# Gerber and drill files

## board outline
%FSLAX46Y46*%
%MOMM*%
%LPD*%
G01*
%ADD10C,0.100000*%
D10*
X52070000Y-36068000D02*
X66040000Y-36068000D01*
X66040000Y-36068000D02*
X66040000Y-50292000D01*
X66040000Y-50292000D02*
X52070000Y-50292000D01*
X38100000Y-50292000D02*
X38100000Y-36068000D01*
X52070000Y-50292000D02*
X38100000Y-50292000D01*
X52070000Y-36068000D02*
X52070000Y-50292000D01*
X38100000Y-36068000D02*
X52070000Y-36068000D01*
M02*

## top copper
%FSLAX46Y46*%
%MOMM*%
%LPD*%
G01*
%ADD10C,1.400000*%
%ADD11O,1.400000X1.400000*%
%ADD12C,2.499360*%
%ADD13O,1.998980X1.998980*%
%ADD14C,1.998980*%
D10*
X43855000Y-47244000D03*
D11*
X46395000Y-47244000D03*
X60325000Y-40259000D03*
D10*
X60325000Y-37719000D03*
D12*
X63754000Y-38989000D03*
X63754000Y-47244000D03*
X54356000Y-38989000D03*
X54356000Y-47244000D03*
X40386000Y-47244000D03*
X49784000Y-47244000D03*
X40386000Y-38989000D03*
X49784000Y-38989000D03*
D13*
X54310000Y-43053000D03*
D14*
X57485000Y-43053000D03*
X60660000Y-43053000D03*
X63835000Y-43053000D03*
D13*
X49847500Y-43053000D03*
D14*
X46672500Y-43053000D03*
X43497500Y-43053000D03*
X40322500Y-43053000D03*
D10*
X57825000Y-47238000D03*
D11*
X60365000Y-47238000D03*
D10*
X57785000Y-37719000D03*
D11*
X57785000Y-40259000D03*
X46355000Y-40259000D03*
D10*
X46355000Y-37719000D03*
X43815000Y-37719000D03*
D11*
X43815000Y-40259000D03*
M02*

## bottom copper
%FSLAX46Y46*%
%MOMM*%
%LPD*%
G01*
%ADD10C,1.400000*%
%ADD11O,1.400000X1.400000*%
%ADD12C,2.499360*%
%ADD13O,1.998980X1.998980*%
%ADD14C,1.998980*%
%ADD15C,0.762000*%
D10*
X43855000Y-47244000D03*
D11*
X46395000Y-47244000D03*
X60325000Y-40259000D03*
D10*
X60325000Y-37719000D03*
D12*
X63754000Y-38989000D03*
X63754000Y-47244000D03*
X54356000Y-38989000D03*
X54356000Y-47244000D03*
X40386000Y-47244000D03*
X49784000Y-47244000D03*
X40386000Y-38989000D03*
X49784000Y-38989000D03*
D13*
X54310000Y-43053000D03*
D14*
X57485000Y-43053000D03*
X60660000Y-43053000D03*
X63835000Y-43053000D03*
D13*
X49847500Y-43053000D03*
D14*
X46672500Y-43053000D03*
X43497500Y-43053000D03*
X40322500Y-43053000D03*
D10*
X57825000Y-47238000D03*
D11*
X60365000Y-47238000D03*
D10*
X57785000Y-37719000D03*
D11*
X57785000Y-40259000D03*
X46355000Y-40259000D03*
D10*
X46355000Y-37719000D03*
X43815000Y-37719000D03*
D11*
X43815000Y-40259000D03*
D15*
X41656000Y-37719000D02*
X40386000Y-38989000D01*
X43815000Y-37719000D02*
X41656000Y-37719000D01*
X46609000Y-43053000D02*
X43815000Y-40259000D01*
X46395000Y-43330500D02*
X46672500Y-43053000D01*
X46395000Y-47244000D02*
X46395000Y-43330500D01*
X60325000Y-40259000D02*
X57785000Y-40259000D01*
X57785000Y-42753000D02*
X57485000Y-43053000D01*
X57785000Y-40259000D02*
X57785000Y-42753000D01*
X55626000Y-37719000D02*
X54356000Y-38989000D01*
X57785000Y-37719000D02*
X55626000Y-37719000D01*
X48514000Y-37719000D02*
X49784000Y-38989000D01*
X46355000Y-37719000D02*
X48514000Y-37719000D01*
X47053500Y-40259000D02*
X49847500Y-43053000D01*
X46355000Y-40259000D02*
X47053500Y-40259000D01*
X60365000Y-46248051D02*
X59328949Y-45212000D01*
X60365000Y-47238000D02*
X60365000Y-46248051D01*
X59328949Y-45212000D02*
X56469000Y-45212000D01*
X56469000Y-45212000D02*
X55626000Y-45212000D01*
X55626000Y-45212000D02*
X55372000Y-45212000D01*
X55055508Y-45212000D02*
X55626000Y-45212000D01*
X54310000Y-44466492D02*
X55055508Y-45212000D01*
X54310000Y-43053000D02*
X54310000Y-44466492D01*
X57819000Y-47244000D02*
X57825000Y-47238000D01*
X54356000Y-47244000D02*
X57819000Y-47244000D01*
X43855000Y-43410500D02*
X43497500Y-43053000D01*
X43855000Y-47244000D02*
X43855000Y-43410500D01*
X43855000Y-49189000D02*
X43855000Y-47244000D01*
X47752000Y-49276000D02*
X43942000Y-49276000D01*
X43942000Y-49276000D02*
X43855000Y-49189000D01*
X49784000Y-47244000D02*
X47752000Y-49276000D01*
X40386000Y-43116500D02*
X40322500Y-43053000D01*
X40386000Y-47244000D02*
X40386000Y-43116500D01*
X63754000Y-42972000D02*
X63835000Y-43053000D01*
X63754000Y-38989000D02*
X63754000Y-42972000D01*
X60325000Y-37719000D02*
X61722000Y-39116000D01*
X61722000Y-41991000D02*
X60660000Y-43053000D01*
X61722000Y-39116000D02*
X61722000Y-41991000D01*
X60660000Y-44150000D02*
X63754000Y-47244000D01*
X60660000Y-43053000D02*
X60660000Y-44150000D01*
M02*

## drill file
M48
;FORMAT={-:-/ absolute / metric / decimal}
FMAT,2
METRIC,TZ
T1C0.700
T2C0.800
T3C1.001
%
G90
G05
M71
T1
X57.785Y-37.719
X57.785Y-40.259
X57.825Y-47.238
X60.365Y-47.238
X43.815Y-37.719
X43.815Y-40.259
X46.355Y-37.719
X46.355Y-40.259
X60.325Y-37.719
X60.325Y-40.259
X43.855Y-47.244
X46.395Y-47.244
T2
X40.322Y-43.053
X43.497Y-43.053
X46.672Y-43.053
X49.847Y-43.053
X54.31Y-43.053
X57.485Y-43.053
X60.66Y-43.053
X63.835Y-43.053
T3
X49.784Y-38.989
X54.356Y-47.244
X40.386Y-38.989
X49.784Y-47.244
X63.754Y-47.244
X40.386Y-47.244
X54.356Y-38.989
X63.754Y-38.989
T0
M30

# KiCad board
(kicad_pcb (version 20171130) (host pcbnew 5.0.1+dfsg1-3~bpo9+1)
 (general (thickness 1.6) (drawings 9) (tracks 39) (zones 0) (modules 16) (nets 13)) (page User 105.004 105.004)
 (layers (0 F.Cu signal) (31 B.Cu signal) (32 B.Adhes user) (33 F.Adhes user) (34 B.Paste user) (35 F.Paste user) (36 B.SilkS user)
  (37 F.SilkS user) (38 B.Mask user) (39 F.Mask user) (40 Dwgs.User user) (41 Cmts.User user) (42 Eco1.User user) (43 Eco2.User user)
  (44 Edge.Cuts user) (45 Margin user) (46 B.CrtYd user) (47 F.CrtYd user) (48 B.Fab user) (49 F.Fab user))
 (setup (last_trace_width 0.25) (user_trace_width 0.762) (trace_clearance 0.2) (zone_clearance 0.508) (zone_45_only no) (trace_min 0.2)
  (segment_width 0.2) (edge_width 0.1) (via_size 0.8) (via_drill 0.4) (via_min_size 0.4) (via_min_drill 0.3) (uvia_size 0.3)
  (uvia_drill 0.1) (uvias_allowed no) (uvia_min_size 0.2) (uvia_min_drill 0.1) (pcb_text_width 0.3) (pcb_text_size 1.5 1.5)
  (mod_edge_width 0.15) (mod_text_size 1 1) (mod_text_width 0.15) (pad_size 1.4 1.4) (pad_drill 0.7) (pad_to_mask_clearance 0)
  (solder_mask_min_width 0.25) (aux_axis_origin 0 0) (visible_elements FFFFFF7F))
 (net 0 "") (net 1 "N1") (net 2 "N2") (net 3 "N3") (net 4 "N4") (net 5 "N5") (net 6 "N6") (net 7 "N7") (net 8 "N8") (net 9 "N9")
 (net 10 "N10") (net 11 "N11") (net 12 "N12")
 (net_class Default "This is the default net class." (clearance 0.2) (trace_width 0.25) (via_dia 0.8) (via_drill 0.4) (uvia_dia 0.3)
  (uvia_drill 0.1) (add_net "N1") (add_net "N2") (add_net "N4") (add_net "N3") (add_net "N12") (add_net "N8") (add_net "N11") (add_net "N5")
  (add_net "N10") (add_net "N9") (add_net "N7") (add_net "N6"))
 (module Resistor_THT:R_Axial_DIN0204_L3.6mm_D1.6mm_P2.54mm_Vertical (layer F.Cu) (at 43.855 47.244)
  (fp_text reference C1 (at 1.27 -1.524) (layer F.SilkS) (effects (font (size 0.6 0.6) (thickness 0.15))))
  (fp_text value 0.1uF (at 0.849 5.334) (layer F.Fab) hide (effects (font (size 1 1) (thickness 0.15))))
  (pad 1 thru_hole circle (at 0 0) (size 1.4 1.4) (drill 0.7) (layers *.Cu *.Mask) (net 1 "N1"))
  (pad 2 thru_hole oval (at 2.54 0) (size 1.4 1.4) (drill 0.7) (layers *.Cu *.Mask) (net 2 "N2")))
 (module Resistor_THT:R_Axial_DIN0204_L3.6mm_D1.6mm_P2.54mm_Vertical (layer F.Cu) (at 60.325 37.719 270)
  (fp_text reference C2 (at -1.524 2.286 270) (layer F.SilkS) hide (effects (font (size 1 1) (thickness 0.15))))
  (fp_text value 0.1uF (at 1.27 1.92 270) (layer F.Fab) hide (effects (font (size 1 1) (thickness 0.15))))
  (pad 2 thru_hole oval (at 2.54 0 270) (size 1.4 1.4) (drill 0.7) (layers *.Cu *.Mask) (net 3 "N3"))
  (pad 1 thru_hole circle (at 0 0 270) (size 1.4 1.4) (drill 0.7) (layers *.Cu *.Mask) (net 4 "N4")))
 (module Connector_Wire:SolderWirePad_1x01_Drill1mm (layer F.Cu) (at 63.754 38.989)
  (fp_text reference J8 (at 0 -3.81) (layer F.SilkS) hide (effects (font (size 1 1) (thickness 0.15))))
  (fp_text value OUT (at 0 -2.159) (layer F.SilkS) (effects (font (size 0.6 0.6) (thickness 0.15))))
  (pad 1 thru_hole circle (at 0 0) (size 2.49936 2.49936) (drill 1.00076) (layers *.Cu *.Mask) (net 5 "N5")))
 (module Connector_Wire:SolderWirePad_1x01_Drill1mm (layer F.Cu) (at 63.754 47.244)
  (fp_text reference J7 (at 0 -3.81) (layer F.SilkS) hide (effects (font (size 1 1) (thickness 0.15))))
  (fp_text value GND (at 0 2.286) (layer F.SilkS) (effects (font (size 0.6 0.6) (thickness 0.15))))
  (pad 1 thru_hole circle (at 0 0) (size 2.49936 2.49936) (drill 1.00076) (layers *.Cu *.Mask) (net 4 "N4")))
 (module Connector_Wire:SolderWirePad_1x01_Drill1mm (layer F.Cu) (at 54.356 38.989)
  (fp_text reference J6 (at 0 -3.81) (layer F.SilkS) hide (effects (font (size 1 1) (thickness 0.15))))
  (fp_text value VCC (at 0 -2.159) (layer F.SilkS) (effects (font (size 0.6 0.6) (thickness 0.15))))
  (pad 1 thru_hole circle (at 0 0) (size 2.49936 2.49936) (drill 1.00076) (layers *.Cu *.Mask) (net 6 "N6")))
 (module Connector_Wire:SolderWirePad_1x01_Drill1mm (layer F.Cu) (at 54.356 47.244)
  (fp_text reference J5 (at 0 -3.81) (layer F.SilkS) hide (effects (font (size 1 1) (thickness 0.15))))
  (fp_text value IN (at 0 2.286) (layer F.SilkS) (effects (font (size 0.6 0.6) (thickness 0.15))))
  (pad 1 thru_hole circle (at 0 0) (size 2.49936 2.49936) (drill 1.00076) (layers *.Cu *.Mask) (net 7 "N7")))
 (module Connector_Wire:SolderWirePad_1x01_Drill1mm (layer F.Cu) (at 40.386 47.244)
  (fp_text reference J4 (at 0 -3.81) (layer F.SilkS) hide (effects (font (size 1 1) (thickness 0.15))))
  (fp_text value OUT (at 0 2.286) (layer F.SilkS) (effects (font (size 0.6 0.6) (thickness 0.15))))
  (pad 1 thru_hole circle (at 0 0) (size 2.49936 2.49936) (drill 1.00076) (layers *.Cu *.Mask) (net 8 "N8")))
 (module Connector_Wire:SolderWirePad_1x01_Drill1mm (layer F.Cu) (at 49.784 47.244)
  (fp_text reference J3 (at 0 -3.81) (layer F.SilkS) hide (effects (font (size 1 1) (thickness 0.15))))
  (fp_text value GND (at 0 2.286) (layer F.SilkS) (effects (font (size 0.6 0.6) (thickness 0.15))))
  (pad 1 thru_hole circle (at 0 0) (size 2.49936 2.49936) (drill 1.00076) (layers *.Cu *.Mask) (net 1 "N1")))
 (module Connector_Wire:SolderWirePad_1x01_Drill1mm (layer F.Cu) (at 40.386 38.989)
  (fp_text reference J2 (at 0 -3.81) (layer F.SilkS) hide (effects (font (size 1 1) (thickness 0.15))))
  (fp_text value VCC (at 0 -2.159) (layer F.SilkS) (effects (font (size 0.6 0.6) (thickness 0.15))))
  (pad 1 thru_hole circle (at 0 0) (size 2.49936 2.49936) (drill 1.00076) (layers *.Cu *.Mask) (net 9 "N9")))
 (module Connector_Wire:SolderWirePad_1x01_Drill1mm (layer F.Cu) (at 49.784 38.989)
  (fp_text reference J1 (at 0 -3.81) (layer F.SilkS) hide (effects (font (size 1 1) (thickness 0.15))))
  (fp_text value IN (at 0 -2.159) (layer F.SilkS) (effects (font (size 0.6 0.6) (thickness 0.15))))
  (pad 1 thru_hole circle (at 0 0) (size 2.49936 2.49936) (drill 1.00076) (layers *.Cu *.Mask) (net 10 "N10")))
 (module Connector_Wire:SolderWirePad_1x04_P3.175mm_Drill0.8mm (layer F.Cu) (at 54.31 43.053)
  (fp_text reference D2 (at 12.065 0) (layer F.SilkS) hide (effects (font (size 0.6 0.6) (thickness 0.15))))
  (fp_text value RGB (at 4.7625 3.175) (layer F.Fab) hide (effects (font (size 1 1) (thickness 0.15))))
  (pad 1 thru_hole oval (at 0 0) (size 1.99898 1.99898) (drill 0.8001) (layers *.Cu *.Mask) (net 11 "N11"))
  (pad 2 thru_hole circle (at 3.175 0) (size 1.99898 1.99898) (drill 0.8001) (layers *.Cu *.Mask) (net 3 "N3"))
  (pad 3 thru_hole circle (at 6.35 0) (size 1.99898 1.99898) (drill 0.8001) (layers *.Cu *.Mask) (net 4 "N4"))
  (pad 4 thru_hole circle (at 9.525 0) (size 1.99898 1.99898) (drill 0.8001) (layers *.Cu *.Mask) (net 5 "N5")))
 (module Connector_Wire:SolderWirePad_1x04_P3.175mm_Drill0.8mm (layer F.Cu) (at 49.8475 43.053 180)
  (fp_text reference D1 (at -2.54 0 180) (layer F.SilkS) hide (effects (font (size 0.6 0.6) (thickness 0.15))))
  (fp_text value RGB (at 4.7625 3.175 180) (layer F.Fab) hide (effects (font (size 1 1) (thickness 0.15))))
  (pad 1 thru_hole oval (at 0 0 180) (size 1.99898 1.99898) (drill 0.8001) (layers *.Cu *.Mask) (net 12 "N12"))
  (pad 2 thru_hole circle (at 3.175 0 180) (size 1.99898 1.99898) (drill 0.8001) (layers *.Cu *.Mask) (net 2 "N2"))
  (pad 3 thru_hole circle (at 6.35 0 180) (size 1.99898 1.99898) (drill 0.8001) (layers *.Cu *.Mask) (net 1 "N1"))
  (pad 4 thru_hole circle (at 9.525 0 180) (size 1.99898 1.99898) (drill 0.8001) (layers *.Cu *.Mask) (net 8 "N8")))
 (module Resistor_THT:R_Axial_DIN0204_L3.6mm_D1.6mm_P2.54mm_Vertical (layer F.Cu) (at 57.825 47.238)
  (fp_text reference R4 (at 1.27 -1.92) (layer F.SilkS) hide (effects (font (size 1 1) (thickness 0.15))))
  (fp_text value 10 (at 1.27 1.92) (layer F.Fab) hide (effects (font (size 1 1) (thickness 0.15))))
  (pad 1 thru_hole circle (at 0 0) (size 1.4 1.4) (drill 0.7) (layers *.Cu *.Mask) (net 7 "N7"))
  (pad 2 thru_hole oval (at 2.54 0) (size 1.4 1.4) (drill 0.7) (layers *.Cu *.Mask) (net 11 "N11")))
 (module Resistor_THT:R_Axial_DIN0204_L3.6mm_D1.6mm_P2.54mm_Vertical (layer F.Cu) (at 57.785 37.719 270)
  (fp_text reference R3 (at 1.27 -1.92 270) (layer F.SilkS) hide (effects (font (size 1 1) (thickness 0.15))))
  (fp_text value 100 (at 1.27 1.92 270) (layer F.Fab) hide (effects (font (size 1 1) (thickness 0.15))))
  (pad 1 thru_hole circle (at 0 0 270) (size 1.4 1.4) (drill 0.7) (layers *.Cu *.Mask) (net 6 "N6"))
  (pad 2 thru_hole oval (at 2.54 0 270) (size 1.4 1.4) (drill 0.7) (layers *.Cu *.Mask) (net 3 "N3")))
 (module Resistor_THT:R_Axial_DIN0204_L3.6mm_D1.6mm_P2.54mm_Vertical (layer F.Cu) (at 46.355 37.719 270)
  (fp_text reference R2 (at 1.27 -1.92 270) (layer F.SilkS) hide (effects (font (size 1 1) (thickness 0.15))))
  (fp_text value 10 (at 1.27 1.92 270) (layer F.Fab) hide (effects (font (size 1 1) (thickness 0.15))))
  (pad 2 thru_hole oval (at 2.54 0 270) (size 1.4 1.4) (drill 0.7) (layers *.Cu *.Mask) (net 12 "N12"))
  (pad 1 thru_hole circle (at 0 0 270) (size 1.4 1.4) (drill 0.7) (layers *.Cu *.Mask) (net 10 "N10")))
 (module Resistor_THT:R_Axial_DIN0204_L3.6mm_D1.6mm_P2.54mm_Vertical (layer F.Cu) (at 43.815 37.719 270)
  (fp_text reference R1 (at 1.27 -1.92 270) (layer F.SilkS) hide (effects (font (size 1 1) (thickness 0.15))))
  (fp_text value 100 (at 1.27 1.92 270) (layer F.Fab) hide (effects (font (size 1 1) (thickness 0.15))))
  (pad 1 thru_hole circle (at 0 0 270) (size 1.4 1.4) (drill 0.7) (layers *.Cu *.Mask) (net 9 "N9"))
  (pad 2 thru_hole oval (at 2.54 0 270) (size 1.4 1.4) (drill 0.7) (layers *.Cu *.Mask) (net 2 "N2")))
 (gr_line (start 52.07 36.068) (end 66.04 36.068) (layer Edge.Cuts) (width 0.1))
 (gr_line (start 66.04 36.068) (end 66.04 50.292) (layer Edge.Cuts) (width 0.1))
 (gr_line (start 66.04 50.292) (end 52.07 50.292) (layer Edge.Cuts) (width 0.1))
 (gr_line (start 38.1 50.292) (end 38.1 36.068) (layer Edge.Cuts) (width 0.1))
 (gr_line (start 52.07 50.292) (end 38.1 50.292) (layer Edge.Cuts) (width 0.1))
 (gr_line (start 52.07 36.068) (end 52.07 50.292) (layer Edge.Cuts) (width 0.1))
 (gr_line (start 38.1 36.068) (end 52.07 36.068) (layer Edge.Cuts) (width 0.1))
 (segment (start 41.656 37.719) (end 40.386 38.989) (width 0.762) (layer B.Cu) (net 9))
 (segment (start 43.815 37.719) (end 41.656 37.719) (width 0.762) (layer B.Cu) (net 9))
 (segment (start 46.609 43.053) (end 43.815 40.259) (width 0.762) (layer B.Cu) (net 2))
 (segment (start 46.395 43.3305) (end 46.6725 43.053) (width 0.762) (layer B.Cu) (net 2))
 (segment (start 46.395 47.244) (end 46.395 43.3305) (width 0.762) (layer B.Cu) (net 2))
 (segment (start 60.325 40.259) (end 57.785 40.259) (width 0.762) (layer B.Cu) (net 3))
 (segment (start 57.785 42.753) (end 57.485 43.053) (width 0.762) (layer B.Cu) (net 3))
 (segment (start 57.785 40.259) (end 57.785 42.753) (width 0.762) (layer B.Cu) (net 3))
 (segment (start 55.626 37.719) (end 54.356 38.989) (width 0.762) (layer B.Cu) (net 6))
 (segment (start 57.785 37.719) (end 55.626 37.719) (width 0.762) (layer B.Cu) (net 6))
 (segment (start 48.514 37.719) (end 49.784 38.989) (width 0.762) (layer B.Cu) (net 10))
 (segment (start 46.355 37.719) (end 48.514 37.719) (width 0.762) (layer B.Cu) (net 10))
 (segment (start 47.0535 40.259) (end 49.8475 43.053) (width 0.762) (layer B.Cu) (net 12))
 (segment (start 46.355 40.259) (end 47.0535 40.259) (width 0.762) (layer B.Cu) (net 12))
 (segment (start 60.365 46.248051) (end 59.328949 45.212) (width 0.762) (layer B.Cu) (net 11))
 (segment (start 60.365 47.238) (end 60.365 46.248051) (width 0.762) (layer B.Cu) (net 11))
 (segment (start 59.328949 45.212) (end 56.469 45.212) (width 0.762) (layer B.Cu) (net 11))
 (segment (start 56.469 45.212) (end 55.626 45.212) (width 0.762) (layer B.Cu) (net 11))
 (segment (start 55.626 45.212) (end 55.372 45.212) (width 0.762) (layer B.Cu) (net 11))
 (segment (start 55.055508 45.212) (end 55.626 45.212) (width 0.762) (layer B.Cu) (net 11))
 (segment (start 54.31 44.466492) (end 55.055508 45.212) (width 0.762) (layer B.Cu) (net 11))
 (segment (start 54.31 43.053) (end 54.31 44.466492) (width 0.762) (layer B.Cu) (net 11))
 (segment (start 57.819 47.244) (end 57.825 47.238) (width 0.762) (layer B.Cu) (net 7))
 (segment (start 54.356 47.244) (end 57.819 47.244) (width 0.762) (layer B.Cu) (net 7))
 (segment (start 43.855 43.4105) (end 43.4975 43.053) (width 0.762) (layer B.Cu) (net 1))
 (segment (start 43.855 47.244) (end 43.855 43.4105) (width 0.762) (layer B.Cu) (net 1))
 (segment (start 43.855 49.189) (end 43.855 47.244) (width 0.762) (layer B.Cu) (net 1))
 (segment (start 47.752 49.276) (end 43.942 49.276) (width 0.762) (layer B.Cu) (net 1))
 (segment (start 43.942 49.276) (end 43.855 49.189) (width 0.762) (layer B.Cu) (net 1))
 (segment (start 49.784 47.244) (end 47.752 49.276) (width 0.762) (layer B.Cu) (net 1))
 (segment (start 40.386 43.1165) (end 40.3225 43.053) (width 0.762) (layer B.Cu) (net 8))
 (segment (start 40.386 47.244) (end 40.386 43.1165) (width 0.762) (layer B.Cu) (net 8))
 (segment (start 63.754 42.972) (end 63.835 43.053) (width 0.762) (layer B.Cu) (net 5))
 (segment (start 63.754 38.989) (end 63.754 42.972) (width 0.762) (layer B.Cu) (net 5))
 (segment (start 60.325 37.719) (end 61.722 39.116) (width 0.762) (layer B.Cu) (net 4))
 (segment (start 61.722 41.991) (end 60.66 43.053) (width 0.762) (layer B.Cu) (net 4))
 (segment (start 61.722 39.116) (end 61.722 41.991) (width 0.762) (layer B.Cu) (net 4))
 (segment (start 60.66 44.15) (end 63.754 47.244) (width 0.762) (layer B.Cu) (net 4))
 (segment (start 60.66 43.053) (end 60.66 44.15) (width 0.762) (layer B.Cu) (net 4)))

